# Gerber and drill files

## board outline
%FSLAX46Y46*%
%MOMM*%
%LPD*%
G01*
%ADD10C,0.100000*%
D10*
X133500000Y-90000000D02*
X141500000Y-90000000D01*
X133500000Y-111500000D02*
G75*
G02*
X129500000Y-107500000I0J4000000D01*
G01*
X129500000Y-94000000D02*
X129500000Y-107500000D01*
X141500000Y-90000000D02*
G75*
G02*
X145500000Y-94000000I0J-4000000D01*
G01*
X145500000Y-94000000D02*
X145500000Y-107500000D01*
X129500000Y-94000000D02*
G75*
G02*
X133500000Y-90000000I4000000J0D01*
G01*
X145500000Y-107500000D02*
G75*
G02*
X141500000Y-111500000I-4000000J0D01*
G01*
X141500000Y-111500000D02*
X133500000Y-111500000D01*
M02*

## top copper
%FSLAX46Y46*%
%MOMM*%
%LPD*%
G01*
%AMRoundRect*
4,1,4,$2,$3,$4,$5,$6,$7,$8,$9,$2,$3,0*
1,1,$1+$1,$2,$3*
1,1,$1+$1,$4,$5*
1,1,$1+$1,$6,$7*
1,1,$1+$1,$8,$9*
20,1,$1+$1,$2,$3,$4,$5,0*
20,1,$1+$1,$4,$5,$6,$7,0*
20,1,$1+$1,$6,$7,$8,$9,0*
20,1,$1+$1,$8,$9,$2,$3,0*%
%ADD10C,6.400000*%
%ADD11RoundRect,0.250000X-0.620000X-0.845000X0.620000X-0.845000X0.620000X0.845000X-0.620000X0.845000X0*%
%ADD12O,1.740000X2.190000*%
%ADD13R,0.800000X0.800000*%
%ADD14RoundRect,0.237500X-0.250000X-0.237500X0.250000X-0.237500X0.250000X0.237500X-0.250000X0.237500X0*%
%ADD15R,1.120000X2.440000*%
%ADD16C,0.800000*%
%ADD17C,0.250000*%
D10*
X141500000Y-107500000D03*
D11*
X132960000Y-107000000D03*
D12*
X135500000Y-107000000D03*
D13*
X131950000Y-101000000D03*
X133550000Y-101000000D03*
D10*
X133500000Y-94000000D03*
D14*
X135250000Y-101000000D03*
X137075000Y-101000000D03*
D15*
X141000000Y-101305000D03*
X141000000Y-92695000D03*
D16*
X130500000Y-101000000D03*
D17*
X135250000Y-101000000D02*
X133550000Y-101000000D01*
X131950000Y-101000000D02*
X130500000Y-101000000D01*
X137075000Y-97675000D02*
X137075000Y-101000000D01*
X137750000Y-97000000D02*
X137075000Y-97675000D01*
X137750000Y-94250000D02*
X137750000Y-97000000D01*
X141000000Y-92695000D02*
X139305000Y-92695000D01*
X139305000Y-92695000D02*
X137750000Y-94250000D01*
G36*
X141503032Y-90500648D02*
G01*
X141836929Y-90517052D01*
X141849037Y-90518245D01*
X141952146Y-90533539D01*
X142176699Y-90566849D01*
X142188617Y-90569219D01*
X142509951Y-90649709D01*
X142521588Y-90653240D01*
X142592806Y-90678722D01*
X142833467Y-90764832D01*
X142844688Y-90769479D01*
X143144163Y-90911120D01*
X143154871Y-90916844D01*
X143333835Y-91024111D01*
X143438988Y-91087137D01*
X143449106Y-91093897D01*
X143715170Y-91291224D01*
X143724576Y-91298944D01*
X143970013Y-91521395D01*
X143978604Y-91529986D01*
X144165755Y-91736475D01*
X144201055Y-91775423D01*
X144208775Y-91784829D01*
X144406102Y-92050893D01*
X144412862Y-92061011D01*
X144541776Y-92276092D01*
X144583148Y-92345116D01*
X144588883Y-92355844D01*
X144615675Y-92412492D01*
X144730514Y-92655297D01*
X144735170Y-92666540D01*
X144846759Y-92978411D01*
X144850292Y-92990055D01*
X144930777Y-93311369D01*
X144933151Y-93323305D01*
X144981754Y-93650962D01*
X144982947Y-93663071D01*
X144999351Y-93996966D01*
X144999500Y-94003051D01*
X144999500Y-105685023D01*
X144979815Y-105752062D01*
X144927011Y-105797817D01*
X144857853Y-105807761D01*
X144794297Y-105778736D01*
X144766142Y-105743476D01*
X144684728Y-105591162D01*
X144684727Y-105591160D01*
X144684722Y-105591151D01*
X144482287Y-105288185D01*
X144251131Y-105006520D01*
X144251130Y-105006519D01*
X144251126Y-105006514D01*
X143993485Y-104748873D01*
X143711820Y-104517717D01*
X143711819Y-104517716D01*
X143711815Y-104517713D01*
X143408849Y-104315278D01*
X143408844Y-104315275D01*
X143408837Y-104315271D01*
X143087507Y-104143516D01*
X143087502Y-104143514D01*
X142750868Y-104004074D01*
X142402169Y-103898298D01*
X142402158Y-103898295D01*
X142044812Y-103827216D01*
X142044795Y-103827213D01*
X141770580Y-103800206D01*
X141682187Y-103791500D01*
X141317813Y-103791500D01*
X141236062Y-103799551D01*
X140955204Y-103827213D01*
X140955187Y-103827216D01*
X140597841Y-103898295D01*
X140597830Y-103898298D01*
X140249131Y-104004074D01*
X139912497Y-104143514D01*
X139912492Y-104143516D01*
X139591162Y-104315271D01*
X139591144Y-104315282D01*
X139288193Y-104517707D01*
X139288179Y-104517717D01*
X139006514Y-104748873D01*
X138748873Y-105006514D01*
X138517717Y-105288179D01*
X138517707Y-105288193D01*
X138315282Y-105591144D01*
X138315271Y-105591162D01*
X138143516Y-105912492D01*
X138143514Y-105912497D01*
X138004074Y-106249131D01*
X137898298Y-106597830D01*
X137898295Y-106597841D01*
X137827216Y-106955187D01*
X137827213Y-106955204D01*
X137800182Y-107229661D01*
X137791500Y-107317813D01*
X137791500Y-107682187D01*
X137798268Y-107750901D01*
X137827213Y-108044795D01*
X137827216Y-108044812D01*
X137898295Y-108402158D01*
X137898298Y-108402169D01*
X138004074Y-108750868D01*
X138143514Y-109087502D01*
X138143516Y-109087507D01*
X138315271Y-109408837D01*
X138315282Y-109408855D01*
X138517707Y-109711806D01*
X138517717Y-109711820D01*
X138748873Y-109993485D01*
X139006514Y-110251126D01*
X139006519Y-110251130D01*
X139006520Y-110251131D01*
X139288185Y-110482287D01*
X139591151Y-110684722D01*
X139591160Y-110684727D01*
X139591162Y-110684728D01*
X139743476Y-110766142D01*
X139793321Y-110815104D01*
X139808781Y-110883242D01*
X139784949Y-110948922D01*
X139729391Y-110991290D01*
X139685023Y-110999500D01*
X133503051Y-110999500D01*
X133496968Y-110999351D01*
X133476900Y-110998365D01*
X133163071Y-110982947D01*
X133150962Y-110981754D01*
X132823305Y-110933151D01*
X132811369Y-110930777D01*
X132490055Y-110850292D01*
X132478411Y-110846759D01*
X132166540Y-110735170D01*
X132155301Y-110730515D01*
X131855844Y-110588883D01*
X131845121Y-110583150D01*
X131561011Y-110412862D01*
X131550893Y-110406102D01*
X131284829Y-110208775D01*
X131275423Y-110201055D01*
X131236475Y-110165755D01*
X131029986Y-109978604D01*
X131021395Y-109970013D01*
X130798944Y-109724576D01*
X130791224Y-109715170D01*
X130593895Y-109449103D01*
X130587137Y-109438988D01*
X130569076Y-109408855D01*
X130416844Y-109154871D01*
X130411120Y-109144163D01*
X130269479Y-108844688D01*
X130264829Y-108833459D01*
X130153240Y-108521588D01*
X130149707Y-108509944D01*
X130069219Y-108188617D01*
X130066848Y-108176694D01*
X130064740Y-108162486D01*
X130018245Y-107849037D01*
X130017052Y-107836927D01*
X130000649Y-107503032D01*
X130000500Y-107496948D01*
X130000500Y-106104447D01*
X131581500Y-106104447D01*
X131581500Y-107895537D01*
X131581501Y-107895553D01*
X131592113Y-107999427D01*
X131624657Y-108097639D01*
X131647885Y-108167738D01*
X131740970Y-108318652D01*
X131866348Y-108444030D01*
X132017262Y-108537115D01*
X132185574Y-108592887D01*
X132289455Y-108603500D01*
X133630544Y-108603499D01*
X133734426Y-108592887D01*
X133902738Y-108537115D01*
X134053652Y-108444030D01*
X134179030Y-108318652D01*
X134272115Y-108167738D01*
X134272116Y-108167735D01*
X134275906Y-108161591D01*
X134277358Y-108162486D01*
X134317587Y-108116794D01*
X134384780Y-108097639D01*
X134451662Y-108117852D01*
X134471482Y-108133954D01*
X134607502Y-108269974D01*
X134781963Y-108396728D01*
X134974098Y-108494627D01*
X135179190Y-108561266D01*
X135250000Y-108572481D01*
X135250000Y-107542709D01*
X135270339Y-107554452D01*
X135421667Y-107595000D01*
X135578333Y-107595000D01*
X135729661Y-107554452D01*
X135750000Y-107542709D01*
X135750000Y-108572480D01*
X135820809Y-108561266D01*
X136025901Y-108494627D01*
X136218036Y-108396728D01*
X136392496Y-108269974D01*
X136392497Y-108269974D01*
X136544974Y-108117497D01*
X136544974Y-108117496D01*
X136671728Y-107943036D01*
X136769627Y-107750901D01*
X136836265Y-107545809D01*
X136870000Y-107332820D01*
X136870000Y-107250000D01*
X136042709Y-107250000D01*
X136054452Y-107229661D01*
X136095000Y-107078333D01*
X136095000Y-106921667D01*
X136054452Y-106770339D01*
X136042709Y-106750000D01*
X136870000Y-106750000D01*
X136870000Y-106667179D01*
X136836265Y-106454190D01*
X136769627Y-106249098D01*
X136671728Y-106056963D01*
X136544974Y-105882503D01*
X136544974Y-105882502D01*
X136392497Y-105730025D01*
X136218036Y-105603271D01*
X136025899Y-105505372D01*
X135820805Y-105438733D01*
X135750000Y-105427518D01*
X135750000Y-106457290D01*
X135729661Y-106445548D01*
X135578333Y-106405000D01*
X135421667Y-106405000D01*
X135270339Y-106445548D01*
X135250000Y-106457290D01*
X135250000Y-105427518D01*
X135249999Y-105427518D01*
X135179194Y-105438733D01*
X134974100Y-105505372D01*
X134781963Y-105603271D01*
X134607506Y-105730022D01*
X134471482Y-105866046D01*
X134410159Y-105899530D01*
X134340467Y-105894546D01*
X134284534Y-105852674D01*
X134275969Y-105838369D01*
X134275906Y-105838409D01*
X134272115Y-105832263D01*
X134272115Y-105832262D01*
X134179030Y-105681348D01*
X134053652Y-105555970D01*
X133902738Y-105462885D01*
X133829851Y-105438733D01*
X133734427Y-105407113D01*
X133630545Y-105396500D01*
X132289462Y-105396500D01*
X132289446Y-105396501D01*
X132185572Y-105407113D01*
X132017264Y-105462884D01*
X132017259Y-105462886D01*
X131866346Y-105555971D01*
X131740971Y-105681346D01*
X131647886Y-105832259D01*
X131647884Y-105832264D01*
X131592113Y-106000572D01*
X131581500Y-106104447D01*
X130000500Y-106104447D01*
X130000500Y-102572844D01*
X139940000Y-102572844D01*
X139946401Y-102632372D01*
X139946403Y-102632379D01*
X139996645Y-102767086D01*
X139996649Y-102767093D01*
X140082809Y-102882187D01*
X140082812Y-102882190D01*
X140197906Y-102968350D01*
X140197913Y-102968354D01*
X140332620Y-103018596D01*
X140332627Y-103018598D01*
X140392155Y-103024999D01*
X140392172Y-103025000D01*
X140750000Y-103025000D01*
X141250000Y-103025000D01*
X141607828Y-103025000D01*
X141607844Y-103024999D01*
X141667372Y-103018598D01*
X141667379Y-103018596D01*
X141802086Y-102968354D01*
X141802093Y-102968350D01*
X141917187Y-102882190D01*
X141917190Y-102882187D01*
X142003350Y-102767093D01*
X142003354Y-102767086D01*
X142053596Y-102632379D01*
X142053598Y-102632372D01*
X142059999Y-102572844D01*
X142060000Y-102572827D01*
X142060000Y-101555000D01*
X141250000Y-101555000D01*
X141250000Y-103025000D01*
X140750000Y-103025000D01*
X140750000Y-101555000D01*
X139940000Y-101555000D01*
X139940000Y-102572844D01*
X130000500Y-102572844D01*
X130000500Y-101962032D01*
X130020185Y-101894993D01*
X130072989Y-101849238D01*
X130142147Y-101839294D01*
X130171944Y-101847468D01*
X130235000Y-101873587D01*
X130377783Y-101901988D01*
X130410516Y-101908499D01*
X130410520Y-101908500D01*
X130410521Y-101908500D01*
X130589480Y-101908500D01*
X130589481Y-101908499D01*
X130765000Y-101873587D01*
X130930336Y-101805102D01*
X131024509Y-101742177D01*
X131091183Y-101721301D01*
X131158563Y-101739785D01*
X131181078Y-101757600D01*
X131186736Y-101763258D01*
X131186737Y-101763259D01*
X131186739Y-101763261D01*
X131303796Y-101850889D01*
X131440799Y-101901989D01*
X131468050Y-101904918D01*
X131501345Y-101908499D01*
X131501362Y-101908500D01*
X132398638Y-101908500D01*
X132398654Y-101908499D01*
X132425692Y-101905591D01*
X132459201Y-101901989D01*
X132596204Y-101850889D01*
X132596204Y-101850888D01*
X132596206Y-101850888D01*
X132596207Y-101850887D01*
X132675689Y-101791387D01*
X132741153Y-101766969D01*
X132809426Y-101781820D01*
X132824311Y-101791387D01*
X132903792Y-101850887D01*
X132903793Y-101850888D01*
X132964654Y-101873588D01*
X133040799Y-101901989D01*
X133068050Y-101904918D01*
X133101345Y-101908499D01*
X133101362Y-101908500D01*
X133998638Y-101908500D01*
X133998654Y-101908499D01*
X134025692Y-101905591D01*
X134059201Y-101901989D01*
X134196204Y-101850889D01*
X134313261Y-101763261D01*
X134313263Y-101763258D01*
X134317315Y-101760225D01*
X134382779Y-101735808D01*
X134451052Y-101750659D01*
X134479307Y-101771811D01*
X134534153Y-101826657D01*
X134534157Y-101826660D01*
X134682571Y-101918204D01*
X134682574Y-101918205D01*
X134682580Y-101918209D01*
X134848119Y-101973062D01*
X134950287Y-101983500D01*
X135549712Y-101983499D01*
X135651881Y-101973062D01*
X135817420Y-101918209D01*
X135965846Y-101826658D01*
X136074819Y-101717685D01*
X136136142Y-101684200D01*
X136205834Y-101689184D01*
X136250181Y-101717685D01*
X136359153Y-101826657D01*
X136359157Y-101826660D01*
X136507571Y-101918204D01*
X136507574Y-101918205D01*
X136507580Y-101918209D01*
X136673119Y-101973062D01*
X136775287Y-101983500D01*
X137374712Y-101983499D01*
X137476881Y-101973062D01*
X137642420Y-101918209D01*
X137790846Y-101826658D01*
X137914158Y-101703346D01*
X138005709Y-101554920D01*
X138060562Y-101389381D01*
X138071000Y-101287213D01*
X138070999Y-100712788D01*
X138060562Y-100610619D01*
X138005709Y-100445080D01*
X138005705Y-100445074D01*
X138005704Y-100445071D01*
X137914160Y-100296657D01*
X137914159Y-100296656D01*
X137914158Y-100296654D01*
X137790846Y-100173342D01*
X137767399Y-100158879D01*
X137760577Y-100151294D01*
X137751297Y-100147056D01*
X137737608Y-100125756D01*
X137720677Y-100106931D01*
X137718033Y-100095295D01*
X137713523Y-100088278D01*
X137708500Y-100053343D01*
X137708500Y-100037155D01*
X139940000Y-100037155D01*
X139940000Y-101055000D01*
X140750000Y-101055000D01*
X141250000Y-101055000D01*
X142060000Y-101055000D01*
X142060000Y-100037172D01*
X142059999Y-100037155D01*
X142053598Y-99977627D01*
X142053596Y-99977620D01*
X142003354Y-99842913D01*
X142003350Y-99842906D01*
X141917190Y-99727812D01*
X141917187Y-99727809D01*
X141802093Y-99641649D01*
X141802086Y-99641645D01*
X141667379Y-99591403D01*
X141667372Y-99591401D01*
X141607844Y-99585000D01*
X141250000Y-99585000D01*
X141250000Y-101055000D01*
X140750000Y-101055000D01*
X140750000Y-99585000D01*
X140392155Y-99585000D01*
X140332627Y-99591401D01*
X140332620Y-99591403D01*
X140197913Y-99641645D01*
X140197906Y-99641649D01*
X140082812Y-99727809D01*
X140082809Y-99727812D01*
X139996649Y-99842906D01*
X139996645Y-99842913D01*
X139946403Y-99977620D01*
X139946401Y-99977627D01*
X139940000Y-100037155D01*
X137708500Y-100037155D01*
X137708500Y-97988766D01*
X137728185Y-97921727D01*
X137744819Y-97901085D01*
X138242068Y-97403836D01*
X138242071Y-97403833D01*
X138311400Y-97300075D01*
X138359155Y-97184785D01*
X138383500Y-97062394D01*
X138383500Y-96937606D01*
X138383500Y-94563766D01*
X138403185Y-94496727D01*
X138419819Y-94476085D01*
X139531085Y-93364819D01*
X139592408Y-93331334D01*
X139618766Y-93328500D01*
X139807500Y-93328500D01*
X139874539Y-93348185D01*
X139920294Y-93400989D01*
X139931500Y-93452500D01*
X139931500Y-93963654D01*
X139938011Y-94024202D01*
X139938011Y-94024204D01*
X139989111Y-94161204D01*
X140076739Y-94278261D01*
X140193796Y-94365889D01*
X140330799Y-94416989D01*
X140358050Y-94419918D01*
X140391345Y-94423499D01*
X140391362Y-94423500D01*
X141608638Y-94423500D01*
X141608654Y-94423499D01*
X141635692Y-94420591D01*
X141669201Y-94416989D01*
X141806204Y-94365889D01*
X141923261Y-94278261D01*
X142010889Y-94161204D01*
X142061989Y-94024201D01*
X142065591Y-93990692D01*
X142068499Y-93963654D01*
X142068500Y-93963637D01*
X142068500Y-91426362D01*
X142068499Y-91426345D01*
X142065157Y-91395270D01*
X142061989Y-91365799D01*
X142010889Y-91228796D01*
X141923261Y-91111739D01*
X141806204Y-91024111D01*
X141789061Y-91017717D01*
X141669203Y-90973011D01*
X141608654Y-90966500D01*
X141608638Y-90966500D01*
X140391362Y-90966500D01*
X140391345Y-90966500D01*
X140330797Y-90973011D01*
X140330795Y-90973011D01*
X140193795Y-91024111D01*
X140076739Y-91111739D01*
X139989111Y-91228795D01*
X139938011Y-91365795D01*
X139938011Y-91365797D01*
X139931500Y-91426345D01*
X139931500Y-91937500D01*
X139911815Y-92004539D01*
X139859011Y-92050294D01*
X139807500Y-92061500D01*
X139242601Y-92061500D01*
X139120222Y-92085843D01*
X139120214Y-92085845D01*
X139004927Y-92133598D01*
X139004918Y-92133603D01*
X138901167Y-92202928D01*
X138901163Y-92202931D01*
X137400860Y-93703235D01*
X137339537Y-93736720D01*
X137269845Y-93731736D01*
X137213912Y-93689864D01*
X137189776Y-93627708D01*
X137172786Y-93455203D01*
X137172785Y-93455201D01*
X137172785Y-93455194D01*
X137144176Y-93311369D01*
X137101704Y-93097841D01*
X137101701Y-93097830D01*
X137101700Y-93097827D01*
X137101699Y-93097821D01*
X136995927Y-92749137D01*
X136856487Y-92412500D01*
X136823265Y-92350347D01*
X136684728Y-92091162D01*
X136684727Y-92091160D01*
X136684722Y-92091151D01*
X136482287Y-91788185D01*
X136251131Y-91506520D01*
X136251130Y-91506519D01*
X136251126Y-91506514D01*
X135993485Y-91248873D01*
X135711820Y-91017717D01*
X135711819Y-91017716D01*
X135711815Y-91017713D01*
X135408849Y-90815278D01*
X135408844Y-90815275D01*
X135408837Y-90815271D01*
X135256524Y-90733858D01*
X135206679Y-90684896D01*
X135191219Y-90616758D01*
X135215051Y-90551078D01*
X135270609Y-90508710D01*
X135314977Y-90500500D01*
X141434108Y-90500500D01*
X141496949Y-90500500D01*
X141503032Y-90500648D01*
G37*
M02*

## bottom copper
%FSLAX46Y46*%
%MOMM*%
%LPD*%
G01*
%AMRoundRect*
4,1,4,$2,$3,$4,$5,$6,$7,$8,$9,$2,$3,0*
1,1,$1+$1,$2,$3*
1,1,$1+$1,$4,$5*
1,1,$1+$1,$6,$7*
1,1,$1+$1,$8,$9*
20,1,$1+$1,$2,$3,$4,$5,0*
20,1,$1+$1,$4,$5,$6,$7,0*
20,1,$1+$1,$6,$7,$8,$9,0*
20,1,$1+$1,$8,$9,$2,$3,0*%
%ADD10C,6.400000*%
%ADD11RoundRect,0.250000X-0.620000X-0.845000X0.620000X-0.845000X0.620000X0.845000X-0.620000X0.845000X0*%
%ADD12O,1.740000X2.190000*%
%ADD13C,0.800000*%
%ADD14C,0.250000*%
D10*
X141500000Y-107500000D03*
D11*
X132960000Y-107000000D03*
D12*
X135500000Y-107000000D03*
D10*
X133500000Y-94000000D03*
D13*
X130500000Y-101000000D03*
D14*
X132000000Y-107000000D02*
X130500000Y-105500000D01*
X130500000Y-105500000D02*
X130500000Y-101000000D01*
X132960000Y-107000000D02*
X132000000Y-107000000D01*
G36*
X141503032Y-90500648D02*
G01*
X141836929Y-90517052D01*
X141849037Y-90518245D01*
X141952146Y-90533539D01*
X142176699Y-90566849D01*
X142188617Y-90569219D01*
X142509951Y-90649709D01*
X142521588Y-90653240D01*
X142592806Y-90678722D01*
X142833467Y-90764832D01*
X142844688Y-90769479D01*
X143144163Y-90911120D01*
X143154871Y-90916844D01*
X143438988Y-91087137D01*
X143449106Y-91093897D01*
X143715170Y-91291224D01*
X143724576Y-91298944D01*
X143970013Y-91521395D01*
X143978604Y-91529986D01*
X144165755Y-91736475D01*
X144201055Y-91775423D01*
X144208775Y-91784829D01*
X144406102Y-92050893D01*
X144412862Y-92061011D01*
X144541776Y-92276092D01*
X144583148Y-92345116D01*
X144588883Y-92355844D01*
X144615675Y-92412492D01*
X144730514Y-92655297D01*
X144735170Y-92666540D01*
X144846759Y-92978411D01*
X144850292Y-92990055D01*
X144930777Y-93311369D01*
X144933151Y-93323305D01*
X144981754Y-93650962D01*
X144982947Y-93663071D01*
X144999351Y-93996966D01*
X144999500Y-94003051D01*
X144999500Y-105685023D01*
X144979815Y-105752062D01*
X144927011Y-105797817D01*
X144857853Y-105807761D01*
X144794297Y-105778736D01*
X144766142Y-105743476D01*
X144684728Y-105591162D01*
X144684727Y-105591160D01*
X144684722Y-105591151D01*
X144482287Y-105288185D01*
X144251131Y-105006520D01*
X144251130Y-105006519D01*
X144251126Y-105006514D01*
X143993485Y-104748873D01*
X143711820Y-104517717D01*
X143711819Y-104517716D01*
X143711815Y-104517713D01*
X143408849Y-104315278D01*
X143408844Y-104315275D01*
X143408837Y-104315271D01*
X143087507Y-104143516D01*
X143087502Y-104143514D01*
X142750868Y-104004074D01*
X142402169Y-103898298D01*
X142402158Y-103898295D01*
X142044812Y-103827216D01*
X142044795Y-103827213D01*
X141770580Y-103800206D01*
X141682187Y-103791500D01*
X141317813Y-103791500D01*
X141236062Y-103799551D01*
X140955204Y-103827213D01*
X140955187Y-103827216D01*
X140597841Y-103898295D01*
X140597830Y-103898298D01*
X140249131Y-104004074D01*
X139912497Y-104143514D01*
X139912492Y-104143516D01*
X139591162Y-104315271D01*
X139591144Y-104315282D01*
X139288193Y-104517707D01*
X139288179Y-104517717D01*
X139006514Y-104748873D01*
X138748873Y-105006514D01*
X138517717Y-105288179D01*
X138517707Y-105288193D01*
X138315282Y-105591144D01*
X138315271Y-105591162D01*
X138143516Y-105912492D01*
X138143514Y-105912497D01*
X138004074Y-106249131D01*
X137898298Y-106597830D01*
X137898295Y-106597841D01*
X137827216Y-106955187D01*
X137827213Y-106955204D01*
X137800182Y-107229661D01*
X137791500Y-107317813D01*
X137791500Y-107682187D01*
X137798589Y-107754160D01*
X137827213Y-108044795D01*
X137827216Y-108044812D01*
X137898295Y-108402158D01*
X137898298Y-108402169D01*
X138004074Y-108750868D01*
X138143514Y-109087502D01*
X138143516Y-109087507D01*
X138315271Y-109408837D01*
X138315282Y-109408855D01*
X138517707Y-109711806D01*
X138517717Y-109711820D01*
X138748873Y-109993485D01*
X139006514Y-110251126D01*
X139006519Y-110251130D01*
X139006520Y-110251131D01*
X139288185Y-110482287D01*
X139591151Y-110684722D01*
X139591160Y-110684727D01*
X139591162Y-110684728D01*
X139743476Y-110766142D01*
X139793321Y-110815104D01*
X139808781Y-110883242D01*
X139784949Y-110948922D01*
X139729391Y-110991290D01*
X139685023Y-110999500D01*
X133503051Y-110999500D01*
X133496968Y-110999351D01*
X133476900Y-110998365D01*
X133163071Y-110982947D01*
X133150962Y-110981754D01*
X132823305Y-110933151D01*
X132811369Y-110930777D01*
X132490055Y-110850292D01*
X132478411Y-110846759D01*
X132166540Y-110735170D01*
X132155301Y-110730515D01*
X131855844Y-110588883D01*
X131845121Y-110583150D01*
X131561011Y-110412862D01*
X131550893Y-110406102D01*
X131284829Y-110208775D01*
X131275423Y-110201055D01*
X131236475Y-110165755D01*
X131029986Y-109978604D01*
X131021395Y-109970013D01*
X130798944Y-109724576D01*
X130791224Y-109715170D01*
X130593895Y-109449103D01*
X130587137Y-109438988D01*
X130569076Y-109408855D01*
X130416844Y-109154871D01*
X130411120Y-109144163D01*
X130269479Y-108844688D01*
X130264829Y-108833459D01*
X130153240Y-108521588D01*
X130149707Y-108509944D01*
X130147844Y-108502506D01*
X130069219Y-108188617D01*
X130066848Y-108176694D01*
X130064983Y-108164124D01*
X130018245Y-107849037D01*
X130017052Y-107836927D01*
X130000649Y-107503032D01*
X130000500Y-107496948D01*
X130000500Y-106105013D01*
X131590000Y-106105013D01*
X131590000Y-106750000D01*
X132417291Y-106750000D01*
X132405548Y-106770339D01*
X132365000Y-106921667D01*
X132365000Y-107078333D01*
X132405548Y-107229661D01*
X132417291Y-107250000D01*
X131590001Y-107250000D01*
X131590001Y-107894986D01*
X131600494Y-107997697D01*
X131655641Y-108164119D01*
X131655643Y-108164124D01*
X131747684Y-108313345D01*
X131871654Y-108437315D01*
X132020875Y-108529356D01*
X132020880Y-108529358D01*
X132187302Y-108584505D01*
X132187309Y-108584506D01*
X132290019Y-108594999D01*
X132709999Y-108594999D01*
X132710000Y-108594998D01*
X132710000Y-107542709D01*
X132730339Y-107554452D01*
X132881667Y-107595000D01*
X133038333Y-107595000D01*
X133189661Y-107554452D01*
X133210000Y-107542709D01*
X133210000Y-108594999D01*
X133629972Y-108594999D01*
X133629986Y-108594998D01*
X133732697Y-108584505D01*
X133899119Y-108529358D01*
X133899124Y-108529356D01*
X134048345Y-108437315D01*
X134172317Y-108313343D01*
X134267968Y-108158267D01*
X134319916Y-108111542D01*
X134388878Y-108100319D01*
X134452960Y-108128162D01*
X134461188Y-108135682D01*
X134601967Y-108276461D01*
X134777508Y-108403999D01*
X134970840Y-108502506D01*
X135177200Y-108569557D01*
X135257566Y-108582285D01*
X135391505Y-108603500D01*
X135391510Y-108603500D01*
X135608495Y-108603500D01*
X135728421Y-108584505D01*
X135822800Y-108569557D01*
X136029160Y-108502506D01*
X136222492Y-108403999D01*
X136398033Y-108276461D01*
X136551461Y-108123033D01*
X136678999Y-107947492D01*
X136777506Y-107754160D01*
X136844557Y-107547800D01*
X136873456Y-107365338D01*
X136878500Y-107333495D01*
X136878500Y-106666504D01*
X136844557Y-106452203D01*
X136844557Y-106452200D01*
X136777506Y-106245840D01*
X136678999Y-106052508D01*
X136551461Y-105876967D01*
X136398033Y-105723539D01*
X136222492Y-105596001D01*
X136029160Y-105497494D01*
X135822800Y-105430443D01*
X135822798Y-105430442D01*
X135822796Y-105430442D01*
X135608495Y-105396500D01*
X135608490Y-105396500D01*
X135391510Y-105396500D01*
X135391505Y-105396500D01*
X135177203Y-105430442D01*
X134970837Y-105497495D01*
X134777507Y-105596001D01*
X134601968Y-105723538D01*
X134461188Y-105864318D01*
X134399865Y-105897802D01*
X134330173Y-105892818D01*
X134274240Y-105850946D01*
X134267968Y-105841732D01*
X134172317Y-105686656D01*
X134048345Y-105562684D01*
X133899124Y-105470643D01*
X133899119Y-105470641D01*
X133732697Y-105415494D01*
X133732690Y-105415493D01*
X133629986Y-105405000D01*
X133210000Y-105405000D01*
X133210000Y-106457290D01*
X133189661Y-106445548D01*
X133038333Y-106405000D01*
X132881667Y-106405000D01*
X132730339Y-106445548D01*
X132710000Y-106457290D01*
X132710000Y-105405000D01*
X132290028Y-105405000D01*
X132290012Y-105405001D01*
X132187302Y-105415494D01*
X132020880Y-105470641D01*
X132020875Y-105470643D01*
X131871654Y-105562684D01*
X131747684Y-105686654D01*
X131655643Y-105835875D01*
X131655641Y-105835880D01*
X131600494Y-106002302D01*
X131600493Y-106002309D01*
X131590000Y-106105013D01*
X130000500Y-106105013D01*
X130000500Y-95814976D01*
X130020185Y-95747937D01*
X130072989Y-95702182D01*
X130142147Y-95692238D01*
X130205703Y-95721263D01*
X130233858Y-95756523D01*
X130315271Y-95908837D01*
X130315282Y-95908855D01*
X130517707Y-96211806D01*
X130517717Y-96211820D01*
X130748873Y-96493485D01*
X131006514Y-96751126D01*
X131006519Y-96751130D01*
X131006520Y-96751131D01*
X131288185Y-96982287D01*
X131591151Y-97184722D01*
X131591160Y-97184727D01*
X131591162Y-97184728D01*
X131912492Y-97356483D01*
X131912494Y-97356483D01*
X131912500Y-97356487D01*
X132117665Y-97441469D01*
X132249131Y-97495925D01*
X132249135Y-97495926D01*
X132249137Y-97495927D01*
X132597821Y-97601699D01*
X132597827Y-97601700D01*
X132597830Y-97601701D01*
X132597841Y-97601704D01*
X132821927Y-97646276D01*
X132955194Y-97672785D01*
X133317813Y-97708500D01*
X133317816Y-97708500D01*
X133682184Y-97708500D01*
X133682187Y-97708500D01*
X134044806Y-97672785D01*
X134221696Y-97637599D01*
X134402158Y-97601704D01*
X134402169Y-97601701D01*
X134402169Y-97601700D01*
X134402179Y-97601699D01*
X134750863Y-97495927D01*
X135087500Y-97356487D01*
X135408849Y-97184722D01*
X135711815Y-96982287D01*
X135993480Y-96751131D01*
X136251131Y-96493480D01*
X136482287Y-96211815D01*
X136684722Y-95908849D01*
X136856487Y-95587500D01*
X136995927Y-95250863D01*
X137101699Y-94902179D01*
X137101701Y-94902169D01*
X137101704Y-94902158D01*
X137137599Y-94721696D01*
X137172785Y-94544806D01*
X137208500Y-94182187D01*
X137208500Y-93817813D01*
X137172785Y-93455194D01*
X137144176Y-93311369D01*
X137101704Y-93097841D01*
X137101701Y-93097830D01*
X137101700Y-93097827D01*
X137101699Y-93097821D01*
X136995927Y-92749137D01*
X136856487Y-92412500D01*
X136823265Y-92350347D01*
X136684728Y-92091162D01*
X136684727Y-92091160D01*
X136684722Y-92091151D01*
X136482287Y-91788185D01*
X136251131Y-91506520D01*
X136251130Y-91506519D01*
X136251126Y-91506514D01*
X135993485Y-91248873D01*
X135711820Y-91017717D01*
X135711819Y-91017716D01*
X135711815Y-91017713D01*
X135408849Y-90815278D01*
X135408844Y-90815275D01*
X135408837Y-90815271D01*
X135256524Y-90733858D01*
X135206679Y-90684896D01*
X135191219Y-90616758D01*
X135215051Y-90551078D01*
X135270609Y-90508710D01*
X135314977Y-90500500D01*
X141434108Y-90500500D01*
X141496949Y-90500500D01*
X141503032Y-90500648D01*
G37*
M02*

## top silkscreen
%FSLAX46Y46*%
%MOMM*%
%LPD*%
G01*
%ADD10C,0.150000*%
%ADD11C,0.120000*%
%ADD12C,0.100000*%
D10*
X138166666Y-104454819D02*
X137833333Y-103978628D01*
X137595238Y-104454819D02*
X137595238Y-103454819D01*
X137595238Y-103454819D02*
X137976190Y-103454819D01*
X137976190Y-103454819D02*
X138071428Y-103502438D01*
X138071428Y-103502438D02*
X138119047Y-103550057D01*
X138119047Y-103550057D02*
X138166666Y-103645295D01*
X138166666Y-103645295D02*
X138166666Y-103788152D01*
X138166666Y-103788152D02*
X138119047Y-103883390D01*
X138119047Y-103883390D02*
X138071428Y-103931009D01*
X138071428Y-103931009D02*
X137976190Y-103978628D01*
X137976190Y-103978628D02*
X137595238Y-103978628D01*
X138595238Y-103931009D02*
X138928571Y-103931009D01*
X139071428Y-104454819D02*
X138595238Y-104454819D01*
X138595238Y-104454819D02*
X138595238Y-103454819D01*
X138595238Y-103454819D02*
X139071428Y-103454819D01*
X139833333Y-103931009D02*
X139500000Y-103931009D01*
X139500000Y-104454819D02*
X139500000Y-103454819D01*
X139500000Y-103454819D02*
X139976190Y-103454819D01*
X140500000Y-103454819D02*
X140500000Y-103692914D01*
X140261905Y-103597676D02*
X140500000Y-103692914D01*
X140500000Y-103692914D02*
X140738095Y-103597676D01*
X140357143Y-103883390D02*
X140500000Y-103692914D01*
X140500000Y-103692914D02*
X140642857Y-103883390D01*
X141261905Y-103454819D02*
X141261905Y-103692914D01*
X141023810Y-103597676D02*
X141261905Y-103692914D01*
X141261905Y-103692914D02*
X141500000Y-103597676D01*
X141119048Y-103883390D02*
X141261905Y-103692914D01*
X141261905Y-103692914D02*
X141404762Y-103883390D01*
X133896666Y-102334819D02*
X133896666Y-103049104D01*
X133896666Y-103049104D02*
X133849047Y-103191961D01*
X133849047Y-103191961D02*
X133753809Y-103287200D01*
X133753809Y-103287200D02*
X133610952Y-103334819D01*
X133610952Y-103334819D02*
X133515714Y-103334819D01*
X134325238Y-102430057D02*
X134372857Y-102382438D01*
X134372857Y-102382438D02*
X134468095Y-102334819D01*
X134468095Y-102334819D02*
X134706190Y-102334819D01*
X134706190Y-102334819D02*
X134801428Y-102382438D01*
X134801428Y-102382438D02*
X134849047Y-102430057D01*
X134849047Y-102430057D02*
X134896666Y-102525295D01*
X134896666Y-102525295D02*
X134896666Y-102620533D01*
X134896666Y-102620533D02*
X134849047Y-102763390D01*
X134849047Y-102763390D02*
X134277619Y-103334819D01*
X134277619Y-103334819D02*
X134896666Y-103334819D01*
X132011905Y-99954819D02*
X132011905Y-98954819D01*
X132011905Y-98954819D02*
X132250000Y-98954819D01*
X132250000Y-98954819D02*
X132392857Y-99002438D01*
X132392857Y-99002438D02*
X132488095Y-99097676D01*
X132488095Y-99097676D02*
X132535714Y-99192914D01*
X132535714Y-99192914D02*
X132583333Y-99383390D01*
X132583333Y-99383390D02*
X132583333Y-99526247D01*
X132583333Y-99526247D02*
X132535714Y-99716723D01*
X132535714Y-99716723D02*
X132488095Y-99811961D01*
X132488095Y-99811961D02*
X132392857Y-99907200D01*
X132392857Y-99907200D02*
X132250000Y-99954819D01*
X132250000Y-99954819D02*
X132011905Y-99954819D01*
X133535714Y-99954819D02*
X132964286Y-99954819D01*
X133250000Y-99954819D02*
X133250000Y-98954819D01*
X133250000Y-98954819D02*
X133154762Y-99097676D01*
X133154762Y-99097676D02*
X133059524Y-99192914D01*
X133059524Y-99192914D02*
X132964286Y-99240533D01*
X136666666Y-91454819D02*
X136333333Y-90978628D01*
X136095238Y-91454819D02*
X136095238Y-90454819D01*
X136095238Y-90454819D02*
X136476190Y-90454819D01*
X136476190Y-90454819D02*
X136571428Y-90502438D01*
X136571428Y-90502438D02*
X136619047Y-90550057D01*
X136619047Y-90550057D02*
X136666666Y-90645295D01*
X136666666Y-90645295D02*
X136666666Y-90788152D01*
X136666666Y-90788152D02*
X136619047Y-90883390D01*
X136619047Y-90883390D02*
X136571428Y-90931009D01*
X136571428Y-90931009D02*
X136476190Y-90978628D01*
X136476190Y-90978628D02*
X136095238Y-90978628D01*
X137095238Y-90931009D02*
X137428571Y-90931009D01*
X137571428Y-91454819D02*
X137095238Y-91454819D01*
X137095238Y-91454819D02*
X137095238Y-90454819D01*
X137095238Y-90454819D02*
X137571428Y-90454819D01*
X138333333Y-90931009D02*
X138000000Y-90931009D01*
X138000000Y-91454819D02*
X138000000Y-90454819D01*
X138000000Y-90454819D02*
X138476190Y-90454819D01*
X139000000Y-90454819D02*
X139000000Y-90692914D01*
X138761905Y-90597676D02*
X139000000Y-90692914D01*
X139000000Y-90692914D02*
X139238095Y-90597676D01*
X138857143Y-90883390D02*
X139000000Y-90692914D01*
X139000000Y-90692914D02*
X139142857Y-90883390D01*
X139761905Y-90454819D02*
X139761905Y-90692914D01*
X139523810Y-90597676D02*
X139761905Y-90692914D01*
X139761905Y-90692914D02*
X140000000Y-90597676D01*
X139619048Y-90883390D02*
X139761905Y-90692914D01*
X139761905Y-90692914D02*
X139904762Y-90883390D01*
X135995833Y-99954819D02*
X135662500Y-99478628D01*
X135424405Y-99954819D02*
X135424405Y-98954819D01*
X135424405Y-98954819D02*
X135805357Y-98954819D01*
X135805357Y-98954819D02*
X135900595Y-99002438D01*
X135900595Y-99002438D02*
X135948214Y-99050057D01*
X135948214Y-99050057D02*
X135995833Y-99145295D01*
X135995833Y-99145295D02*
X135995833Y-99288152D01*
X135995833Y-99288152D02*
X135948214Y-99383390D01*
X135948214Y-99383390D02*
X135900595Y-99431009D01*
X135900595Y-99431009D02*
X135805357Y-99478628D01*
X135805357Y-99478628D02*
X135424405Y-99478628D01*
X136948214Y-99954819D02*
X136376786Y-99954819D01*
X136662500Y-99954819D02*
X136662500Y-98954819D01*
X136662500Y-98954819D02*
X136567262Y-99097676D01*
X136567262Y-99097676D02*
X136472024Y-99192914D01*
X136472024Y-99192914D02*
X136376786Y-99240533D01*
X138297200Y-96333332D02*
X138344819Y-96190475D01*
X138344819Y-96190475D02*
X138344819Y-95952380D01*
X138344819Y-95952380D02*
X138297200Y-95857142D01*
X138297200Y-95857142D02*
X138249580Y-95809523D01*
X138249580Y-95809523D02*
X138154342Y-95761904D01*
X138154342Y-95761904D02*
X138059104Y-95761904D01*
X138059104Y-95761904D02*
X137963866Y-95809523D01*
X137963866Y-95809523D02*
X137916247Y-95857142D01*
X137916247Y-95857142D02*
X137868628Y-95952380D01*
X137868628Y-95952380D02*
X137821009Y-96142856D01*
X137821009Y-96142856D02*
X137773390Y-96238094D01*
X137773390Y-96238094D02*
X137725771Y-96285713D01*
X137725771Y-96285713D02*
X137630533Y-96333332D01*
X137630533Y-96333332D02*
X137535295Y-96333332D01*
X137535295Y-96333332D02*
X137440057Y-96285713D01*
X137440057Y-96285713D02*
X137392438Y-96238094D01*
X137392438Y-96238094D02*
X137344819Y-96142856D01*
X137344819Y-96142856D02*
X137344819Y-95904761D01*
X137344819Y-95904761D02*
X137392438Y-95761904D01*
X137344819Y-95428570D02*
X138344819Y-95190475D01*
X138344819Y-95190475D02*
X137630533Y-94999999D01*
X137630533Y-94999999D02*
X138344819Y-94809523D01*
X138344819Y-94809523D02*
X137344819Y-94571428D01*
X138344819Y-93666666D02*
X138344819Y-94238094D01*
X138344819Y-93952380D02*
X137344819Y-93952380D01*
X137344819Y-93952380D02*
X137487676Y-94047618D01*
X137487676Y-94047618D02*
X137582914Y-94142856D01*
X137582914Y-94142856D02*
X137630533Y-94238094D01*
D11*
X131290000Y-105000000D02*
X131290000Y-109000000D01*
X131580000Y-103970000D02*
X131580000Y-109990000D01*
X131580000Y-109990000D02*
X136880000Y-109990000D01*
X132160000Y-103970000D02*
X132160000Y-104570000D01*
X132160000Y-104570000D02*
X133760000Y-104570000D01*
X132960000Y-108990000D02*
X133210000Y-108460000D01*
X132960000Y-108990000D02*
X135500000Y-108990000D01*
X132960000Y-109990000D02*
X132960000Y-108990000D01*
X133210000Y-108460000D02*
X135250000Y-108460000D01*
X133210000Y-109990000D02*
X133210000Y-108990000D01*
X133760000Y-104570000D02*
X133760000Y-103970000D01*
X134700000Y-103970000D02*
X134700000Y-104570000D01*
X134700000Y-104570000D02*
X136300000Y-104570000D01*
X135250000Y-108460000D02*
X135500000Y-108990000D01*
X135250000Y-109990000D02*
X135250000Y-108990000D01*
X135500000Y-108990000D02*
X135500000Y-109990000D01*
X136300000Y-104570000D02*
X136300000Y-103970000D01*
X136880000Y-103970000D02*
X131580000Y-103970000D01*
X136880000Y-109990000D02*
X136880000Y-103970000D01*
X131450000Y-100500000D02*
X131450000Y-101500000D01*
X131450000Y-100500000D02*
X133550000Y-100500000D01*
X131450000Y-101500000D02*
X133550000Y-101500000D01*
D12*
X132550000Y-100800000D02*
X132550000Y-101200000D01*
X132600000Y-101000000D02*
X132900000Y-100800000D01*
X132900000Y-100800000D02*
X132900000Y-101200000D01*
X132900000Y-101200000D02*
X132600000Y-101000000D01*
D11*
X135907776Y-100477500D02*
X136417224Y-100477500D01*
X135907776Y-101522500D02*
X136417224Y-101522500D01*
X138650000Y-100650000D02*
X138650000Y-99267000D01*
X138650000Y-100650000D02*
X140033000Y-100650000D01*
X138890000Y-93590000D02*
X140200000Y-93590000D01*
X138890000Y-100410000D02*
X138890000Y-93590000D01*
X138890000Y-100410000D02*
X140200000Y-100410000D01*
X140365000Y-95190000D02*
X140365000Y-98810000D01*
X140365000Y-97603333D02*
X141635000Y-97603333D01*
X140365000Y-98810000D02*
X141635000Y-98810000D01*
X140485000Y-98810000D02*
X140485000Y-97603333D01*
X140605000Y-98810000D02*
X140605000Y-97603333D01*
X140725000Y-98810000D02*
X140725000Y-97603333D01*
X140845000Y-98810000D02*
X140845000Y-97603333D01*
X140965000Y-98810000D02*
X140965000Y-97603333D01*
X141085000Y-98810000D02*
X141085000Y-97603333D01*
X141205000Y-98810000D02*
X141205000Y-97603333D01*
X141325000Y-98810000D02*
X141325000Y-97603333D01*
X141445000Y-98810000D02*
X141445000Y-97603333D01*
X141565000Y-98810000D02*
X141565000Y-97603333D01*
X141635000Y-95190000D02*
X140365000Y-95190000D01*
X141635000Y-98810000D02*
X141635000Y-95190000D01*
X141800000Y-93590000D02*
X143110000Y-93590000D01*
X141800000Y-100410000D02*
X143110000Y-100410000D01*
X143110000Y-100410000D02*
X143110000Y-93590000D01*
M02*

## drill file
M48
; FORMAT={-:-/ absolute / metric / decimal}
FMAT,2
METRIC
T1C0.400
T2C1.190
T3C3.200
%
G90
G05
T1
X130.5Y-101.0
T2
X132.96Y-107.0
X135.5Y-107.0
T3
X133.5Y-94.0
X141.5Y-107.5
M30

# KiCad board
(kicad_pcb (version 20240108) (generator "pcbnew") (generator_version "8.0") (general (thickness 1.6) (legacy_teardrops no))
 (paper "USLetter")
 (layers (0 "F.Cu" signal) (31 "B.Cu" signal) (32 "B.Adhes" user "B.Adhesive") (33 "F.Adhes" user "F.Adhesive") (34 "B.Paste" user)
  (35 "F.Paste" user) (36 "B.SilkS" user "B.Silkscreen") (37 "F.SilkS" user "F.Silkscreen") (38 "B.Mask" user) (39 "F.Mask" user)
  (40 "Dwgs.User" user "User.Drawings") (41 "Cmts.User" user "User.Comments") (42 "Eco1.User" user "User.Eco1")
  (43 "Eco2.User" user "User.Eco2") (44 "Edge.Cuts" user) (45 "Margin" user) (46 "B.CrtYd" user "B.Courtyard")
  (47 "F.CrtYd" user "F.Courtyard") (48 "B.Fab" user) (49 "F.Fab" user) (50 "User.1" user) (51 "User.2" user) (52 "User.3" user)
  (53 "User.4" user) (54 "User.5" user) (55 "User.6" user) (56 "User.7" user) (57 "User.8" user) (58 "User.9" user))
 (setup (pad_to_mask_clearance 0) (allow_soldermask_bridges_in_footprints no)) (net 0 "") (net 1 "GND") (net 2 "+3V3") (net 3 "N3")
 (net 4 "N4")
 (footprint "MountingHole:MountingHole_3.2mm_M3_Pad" (layer "F.Cu") (at 141.5 107.5)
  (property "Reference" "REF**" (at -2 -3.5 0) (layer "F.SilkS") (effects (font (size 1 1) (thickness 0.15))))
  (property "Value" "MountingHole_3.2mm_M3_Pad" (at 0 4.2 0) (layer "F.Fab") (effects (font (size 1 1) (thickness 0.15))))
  (pad "1" thru_hole circle (at 0 0) (size 6.4 6.4) (drill 3.2) (layers "*.Cu" "*.Mask") (remove_unused_layers no)))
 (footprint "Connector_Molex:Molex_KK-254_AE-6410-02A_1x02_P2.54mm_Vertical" (layer "F.Cu") (at 132.96 107)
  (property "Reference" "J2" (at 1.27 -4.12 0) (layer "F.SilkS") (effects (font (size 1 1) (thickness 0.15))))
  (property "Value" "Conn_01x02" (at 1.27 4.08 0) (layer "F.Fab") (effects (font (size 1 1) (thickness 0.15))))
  (fp_line (start -1.67 -2) (end -1.67 2) (stroke (width 0.12) (type solid)) (layer "F.SilkS"))
  (fp_line (start -1.38 -3.03) (end -1.38 2.99) (stroke (width 0.12) (type solid)) (layer "F.SilkS"))
  (fp_line (start -1.38 2.99) (end 3.92 2.99) (stroke (width 0.12) (type solid)) (layer "F.SilkS"))
  (fp_line (start -0.8 -3.03) (end -0.8 -2.43) (stroke (width 0.12) (type solid)) (layer "F.SilkS"))
  (fp_line (start -0.8 -2.43) (end 0.8 -2.43) (stroke (width 0.12) (type solid)) (layer "F.SilkS"))
  (fp_line (start 0 1.99) (end 0.25 1.46) (stroke (width 0.12) (type solid)) (layer "F.SilkS"))
  (fp_line (start 0 1.99) (end 2.54 1.99) (stroke (width 0.12) (type solid)) (layer "F.SilkS"))
  (fp_line (start 0 2.99) (end 0 1.99) (stroke (width 0.12) (type solid)) (layer "F.SilkS"))
  (fp_line (start 0.25 1.46) (end 2.29 1.46) (stroke (width 0.12) (type solid)) (layer "F.SilkS"))
  (fp_line (start 0.25 2.99) (end 0.25 1.99) (stroke (width 0.12) (type solid)) (layer "F.SilkS"))
  (fp_line (start 0.8 -2.43) (end 0.8 -3.03) (stroke (width 0.12) (type solid)) (layer "F.SilkS"))
  (fp_line (start 1.74 -3.03) (end 1.74 -2.43) (stroke (width 0.12) (type solid)) (layer "F.SilkS"))
  (fp_line (start 1.74 -2.43) (end 3.34 -2.43) (stroke (width 0.12) (type solid)) (layer "F.SilkS"))
  (fp_line (start 2.29 1.46) (end 2.54 1.99) (stroke (width 0.12) (type solid)) (layer "F.SilkS"))
  (fp_line (start 2.29 2.99) (end 2.29 1.99) (stroke (width 0.12) (type solid)) (layer "F.SilkS"))
  (fp_line (start 2.54 1.99) (end 2.54 2.99) (stroke (width 0.12) (type solid)) (layer "F.SilkS"))
  (fp_line (start 3.34 -2.43) (end 3.34 -3.03) (stroke (width 0.12) (type solid)) (layer "F.SilkS"))
  (fp_line (start 3.92 -3.03) (end -1.38 -3.03) (stroke (width 0.12) (type solid)) (layer "F.SilkS"))
  (fp_line (start 3.92 2.99) (end 3.92 -3.03) (stroke (width 0.12) (type solid)) (layer "F.SilkS"))
  (pad "1" thru_hole roundrect (at 0 0) (size 1.74 2.19) (drill 1.19) (layers "*.Cu" "*.Mask") (remove_unused_layers no)
   (roundrect_rratio 0.143678) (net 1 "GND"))
  (pad "2" thru_hole oval (at 2.54 0) (size 1.74 2.19) (drill 1.19) (layers "*.Cu" "*.Mask") (remove_unused_layers no) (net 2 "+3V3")))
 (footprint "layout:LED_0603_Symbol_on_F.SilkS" (layer "F.Cu") (at 132.75 101)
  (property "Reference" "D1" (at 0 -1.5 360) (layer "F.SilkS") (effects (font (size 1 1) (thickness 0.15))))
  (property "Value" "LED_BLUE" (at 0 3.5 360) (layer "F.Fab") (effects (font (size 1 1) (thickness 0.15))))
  (fp_line (start -1.3 -0.5) (end -1.3 0.5) (stroke (width 0.12) (type solid)) (layer "F.SilkS"))
  (fp_line (start -1.3 -0.5) (end 0.8 -0.5) (stroke (width 0.12) (type solid)) (layer "F.SilkS"))
  (fp_line (start -1.3 0.5) (end 0.8 0.5) (stroke (width 0.12) (type solid)) (layer "F.SilkS"))
  (fp_line (start -0.2 -0.2) (end -0.2 0.2) (stroke (width 0.1) (type solid)) (layer "F.SilkS"))
  (fp_line (start -0.15 0) (end 0.15 -0.2) (stroke (width 0.1) (type solid)) (layer "F.SilkS"))
  (fp_line (start 0.15 -0.2) (end 0.15 0.2) (stroke (width 0.1) (type solid)) (layer "F.SilkS"))
  (fp_line (start 0.15 0.2) (end -0.15 0) (stroke (width 0.1) (type solid)) (layer "F.SilkS"))
  (pad "1" smd rect (at -0.8 0 180) (size 0.8 0.8) (layers "F.Cu" "F.Paste" "F.Mask") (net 1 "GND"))
  (pad "2" smd rect (at 0.8 0 180) (size 0.8 0.8) (layers "F.Cu" "F.Paste" "F.Mask") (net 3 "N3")))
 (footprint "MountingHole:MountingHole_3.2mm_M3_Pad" (layer "F.Cu") (at 133.5 94)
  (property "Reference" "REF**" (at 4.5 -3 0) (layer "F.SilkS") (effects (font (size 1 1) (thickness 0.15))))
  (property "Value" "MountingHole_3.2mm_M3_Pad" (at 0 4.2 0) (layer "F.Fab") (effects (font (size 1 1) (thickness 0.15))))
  (pad "1" thru_hole circle (at 0 0) (size 6.4 6.4) (drill 3.2) (layers "*.Cu" "*.Mask") (remove_unused_layers no)))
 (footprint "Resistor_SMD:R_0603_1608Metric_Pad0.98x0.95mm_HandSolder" (layer "F.Cu") (at 136.1625 101)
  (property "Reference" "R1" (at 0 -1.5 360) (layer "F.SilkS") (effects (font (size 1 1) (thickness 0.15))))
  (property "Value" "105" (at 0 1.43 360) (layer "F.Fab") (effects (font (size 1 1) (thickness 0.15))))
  (fp_line (start -0.254724 -0.5225) (end 0.254724 -0.5225) (stroke (width 0.12) (type solid)) (layer "F.SilkS"))
  (fp_line (start -0.254724 0.5225) (end 0.254724 0.5225) (stroke (width 0.12) (type solid)) (layer "F.SilkS"))
  (pad "1" smd roundrect (at -0.9125 0) (size 0.975 0.95) (layers "F.Cu" "F.Paste" "F.Mask") (roundrect_rratio 0.25) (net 3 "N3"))
  (pad "2" smd roundrect (at 0.9125 0) (size 0.975 0.95) (layers "F.Cu" "F.Paste" "F.Mask") (roundrect_rratio 0.25) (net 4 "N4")))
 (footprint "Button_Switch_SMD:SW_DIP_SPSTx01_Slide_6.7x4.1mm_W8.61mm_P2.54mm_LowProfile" (layer "F.Cu") (at 141 97 90)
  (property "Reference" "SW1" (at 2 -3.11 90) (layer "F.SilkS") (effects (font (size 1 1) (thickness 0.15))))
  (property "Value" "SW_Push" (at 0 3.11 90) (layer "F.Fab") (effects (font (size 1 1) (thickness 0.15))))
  (fp_line (start -3.65 -2.35) (end -2.267 -2.35) (stroke (width 0.12) (type solid)) (layer "F.SilkS"))
  (fp_line (start -3.65 -2.35) (end -3.65 -0.967) (stroke (width 0.12) (type solid)) (layer "F.SilkS"))
  (fp_line (start 3.41 -2.11) (end 3.41 -0.8) (stroke (width 0.12) (type solid)) (layer "F.SilkS"))
  (fp_line (start -3.41 -2.11) (end 3.41 -2.11) (stroke (width 0.12) (type solid)) (layer "F.SilkS"))
  (fp_line (start -3.41 -2.11) (end -3.41 -0.8) (stroke (width 0.12) (type solid)) (layer "F.SilkS"))
  (fp_line (start 1.81 -0.635) (end -1.81 -0.635) (stroke (width 0.12) (type solid)) (layer "F.SilkS"))
  (fp_line (start -0.603333 -0.635) (end -0.603333 0.635) (stroke (width 0.12) (type solid)) (layer "F.SilkS"))
  (fp_line (start -1.81 -0.635) (end -1.81 0.635) (stroke (width 0.12) (type solid)) (layer "F.SilkS"))
  (fp_line (start -1.81 -0.515) (end -0.603333 -0.515) (stroke (width 0.12) (type solid)) (layer "F.SilkS"))
  (fp_line (start -1.81 -0.395) (end -0.603333 -0.395) (stroke (width 0.12) (type solid)) (layer "F.SilkS"))
  (fp_line (start -1.81 -0.275) (end -0.603333 -0.275) (stroke (width 0.12) (type solid)) (layer "F.SilkS"))
  (fp_line (start -1.81 -0.155) (end -0.603333 -0.155) (stroke (width 0.12) (type solid)) (layer "F.SilkS"))
  (fp_line (start -1.81 -0.035) (end -0.603333 -0.035) (stroke (width 0.12) (type solid)) (layer "F.SilkS"))
  (fp_line (start -1.81 0.085) (end -0.603333 0.085) (stroke (width 0.12) (type solid)) (layer "F.SilkS"))
  (fp_line (start -1.81 0.205) (end -0.603333 0.205) (stroke (width 0.12) (type solid)) (layer "F.SilkS"))
  (fp_line (start -1.81 0.325) (end -0.603333 0.325) (stroke (width 0.12) (type solid)) (layer "F.SilkS"))
  (fp_line (start -1.81 0.445) (end -0.603333 0.445) (stroke (width 0.12) (type solid)) (layer "F.SilkS"))
  (fp_line (start -1.81 0.565) (end -0.603333 0.565) (stroke (width 0.12) (type solid)) (layer "F.SilkS"))
  (fp_line (start 1.81 0.635) (end 1.81 -0.635) (stroke (width 0.12) (type solid)) (layer "F.SilkS"))
  (fp_line (start -1.81 0.635) (end 1.81 0.635) (stroke (width 0.12) (type solid)) (layer "F.SilkS"))
  (fp_line (start 3.41 0.8) (end 3.41 2.11) (stroke (width 0.12) (type solid)) (layer "F.SilkS"))
  (fp_line (start -3.41 0.8) (end -3.41 2.11) (stroke (width 0.12) (type solid)) (layer "F.SilkS"))
  (fp_line (start -3.41 2.11) (end 3.41 2.11) (stroke (width 0.12) (type solid)) (layer "F.SilkS"))
  (pad "1" smd rect (at -4.305 0 90) (size 2.44 1.12) (layers "F.Cu" "F.Paste" "F.Mask") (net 2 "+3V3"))
  (pad "2" smd rect (at 4.305 0 90) (size 2.44 1.12) (layers "F.Cu" "F.Paste" "F.Mask") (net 4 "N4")))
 (gr_line (start 133.5 90) (end 141.5 90) (stroke (width 0.1) (type default)) (layer "Edge.Cuts"))
 (gr_arc (start 133.5 111.5) (mid 130.671573 110.328427) (end 129.5 107.5) (stroke (width 0.1) (type default)) (layer "Edge.Cuts"))
 (gr_line (start 129.5 94) (end 129.5 107.5) (stroke (width 0.1) (type default)) (layer "Edge.Cuts"))
 (gr_arc (start 141.5 90) (mid 144.328427 91.171573) (end 145.5 94) (stroke (width 0.1) (type default)) (layer "Edge.Cuts"))
 (gr_line (start 145.5 94) (end 145.5 107.5) (stroke (width 0.1) (type default)) (layer "Edge.Cuts"))
 (gr_arc (start 129.5 94) (mid 130.671573 91.171573) (end 133.5 90) (stroke (width 0.1) (type default)) (layer "Edge.Cuts"))
 (gr_arc (start 145.5 107.5) (mid 144.328427 110.328427) (end 141.5 111.5) (stroke (width 0.1) (type default)) (layer "Edge.Cuts"))
 (gr_line (start 141.5 111.5) (end 133.5 111.5) (stroke (width 0.1) (type default)) (layer "Edge.Cuts"))
 (segment (start 135.25 101) (end 133.55 101) (width 0.25) (layer "F.Cu") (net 3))
 (segment (start 131.95 101) (end 130.5 101) (width 0.25) (layer "F.Cu") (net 1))
 (via (at 130.5 101) (size 0.8) (drill 0.4) (layers "F.Cu" "B.Cu") (free yes) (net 1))
 (segment (start 132 107) (end 130.5 105.5) (width 0.25) (layer "B.Cu") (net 1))
 (segment (start 130.5 105.5) (end 130.5 101) (width 0.25) (layer "B.Cu") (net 1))
 (segment (start 132.96 107) (end 132 107) (width 0.25) (layer "B.Cu") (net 1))
 (segment (start 137.075 97.675) (end 137.075 101) (width 0.25) (layer "F.Cu") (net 4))
 (segment (start 137.75 97) (end 137.075 97.675) (width 0.25) (layer "F.Cu") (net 4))
 (segment (start 137.75 94.25) (end 137.75 97) (width 0.25) (layer "F.Cu") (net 4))
 (segment (start 141 92.695) (end 139.305 92.695) (width 0.25) (layer "F.Cu") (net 4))
 (segment (start 139.305 92.695) (end 137.75 94.25) (width 0.25) (layer "F.Cu") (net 4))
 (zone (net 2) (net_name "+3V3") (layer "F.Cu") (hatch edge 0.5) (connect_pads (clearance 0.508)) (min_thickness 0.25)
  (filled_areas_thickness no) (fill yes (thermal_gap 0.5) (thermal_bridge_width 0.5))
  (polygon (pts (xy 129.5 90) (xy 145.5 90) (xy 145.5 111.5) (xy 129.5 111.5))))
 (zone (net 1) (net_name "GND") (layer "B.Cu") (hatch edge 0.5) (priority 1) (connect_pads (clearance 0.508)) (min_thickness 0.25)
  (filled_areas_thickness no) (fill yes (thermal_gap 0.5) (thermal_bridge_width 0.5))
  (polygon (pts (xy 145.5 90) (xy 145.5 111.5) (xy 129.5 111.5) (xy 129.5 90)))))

